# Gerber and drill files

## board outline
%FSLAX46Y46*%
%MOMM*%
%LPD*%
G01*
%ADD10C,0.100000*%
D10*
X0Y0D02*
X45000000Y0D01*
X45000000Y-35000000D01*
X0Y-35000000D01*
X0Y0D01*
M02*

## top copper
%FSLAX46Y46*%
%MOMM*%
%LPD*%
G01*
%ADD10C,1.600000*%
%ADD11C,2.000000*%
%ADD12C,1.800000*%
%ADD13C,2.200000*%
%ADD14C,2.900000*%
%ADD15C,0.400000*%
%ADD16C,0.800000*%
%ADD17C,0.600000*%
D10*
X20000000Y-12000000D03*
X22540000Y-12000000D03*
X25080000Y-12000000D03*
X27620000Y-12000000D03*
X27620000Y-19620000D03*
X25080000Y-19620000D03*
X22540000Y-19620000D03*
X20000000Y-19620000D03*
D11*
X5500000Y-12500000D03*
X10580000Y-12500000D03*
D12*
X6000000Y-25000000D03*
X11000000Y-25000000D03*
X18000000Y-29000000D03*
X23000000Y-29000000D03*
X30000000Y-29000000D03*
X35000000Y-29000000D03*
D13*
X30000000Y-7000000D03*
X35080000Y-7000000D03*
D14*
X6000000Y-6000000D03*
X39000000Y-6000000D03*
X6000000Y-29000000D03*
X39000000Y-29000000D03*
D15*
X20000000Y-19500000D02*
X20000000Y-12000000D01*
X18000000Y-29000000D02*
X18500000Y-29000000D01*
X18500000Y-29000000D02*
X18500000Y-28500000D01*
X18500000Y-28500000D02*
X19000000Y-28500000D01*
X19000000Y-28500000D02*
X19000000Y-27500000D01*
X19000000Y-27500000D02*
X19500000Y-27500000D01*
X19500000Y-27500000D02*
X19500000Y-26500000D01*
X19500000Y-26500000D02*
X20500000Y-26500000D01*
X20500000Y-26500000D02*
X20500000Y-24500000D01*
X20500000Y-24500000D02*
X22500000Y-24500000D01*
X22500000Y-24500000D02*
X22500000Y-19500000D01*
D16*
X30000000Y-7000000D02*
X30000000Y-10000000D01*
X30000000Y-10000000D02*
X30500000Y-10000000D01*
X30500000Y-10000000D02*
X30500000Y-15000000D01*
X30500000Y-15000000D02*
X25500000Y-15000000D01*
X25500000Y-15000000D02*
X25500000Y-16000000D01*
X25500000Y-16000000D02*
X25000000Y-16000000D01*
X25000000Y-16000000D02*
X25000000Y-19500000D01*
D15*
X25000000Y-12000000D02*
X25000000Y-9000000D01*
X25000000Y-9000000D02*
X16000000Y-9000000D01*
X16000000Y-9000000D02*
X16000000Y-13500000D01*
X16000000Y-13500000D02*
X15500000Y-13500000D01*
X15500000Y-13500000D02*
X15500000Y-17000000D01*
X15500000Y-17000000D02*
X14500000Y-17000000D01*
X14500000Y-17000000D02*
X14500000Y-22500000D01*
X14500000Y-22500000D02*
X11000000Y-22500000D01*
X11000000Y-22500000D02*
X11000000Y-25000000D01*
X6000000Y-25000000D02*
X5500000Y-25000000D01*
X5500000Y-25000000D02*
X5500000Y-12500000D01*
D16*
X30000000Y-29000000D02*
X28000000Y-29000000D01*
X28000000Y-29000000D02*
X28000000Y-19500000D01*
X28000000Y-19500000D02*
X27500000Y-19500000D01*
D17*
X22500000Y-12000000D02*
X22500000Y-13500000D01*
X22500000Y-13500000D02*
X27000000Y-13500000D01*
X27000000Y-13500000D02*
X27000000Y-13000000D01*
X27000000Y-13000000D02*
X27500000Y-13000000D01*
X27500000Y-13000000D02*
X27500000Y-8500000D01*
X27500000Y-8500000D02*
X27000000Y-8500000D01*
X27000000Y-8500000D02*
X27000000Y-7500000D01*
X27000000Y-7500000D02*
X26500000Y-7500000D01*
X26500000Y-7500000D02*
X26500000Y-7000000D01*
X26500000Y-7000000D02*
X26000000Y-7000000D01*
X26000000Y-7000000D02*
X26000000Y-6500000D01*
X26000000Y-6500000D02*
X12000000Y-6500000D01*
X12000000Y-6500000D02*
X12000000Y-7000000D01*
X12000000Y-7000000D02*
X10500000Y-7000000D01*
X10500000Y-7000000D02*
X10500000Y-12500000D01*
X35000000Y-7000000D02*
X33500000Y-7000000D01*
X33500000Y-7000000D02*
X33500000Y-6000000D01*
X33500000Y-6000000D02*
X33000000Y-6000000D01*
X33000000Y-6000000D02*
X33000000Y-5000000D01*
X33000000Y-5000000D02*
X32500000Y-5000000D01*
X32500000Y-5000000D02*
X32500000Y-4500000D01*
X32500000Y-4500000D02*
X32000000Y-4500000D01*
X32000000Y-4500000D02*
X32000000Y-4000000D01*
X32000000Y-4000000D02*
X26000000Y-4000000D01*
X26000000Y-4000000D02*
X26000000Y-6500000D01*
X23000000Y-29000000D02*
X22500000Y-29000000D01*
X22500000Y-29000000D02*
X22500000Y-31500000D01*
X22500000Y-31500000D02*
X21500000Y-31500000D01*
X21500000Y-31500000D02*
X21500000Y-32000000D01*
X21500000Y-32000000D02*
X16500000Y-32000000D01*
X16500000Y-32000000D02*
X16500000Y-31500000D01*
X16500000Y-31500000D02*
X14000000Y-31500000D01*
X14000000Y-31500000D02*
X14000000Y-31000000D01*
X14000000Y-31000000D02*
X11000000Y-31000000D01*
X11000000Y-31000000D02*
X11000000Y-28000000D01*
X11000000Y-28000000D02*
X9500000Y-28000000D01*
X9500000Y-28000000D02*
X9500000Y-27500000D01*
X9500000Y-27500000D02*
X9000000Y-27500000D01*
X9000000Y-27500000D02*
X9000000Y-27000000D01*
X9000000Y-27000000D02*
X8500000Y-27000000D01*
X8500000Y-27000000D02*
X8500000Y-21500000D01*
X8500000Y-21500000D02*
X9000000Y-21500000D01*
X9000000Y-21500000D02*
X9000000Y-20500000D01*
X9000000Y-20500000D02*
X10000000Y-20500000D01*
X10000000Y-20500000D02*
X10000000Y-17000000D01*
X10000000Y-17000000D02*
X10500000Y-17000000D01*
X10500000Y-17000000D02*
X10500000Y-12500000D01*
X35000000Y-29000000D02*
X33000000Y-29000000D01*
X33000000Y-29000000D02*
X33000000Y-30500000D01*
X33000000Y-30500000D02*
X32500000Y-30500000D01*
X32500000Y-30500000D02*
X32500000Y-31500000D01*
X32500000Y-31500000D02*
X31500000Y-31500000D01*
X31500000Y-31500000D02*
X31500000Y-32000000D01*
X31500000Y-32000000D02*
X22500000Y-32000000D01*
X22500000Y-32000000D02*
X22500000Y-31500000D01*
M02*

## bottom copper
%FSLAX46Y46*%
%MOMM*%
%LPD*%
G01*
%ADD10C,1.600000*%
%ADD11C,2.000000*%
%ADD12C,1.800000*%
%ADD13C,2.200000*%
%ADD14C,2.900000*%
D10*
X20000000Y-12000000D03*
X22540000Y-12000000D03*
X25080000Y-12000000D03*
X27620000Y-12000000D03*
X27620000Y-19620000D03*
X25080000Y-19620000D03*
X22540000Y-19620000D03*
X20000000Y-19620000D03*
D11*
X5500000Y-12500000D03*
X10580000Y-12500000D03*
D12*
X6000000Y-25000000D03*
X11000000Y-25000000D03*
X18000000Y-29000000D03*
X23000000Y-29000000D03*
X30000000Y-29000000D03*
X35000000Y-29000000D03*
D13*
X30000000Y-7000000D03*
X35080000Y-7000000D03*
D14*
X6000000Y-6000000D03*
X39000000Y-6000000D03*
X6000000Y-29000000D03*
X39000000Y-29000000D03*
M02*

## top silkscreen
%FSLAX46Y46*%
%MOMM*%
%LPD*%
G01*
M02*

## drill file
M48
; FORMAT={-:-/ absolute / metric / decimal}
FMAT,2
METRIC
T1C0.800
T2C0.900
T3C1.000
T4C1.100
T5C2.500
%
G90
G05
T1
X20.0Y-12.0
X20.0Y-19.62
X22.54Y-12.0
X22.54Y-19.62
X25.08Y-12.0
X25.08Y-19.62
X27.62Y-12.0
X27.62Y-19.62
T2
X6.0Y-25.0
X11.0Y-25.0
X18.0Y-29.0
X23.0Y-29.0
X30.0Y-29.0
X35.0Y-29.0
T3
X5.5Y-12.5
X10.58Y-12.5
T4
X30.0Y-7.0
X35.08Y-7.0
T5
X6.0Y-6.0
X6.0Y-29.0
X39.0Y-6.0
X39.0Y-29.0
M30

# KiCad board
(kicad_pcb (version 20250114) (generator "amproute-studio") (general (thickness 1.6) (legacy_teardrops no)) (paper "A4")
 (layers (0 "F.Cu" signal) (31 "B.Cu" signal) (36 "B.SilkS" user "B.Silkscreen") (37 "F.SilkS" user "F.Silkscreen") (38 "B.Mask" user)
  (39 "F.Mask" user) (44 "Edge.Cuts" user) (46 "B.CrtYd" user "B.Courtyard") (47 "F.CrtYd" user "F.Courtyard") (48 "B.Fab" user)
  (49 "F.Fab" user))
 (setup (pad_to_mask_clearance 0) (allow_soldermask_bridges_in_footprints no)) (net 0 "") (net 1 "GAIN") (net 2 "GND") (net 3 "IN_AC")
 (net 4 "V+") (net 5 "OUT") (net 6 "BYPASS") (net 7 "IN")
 (gr_rect (start 0 0) (end 45.0000 35.0000) (stroke (width 0.1) (type default)) (fill none) (layer "Edge.Cuts"))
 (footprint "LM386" (layer "F.Cu") (at 18.0000 10.0000)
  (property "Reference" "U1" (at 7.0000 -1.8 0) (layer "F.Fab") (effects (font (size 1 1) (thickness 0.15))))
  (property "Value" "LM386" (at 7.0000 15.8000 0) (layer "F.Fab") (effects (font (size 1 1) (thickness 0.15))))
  (pad "1" thru_hole circle (at 2.0000 2.0000) (size 1.6000 1.6000) (drill 0.8000) (layers "*.Cu" "*.Mask") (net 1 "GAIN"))
  (pad "2" thru_hole circle (at 4.5400 2.0000) (size 1.6000 1.6000) (drill 0.8000) (layers "*.Cu" "*.Mask") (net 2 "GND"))
  (pad "3" thru_hole circle (at 7.0800 2.0000) (size 1.6000 1.6000) (drill 0.8000) (layers "*.Cu" "*.Mask") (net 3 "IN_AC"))
  (pad "4" thru_hole circle (at 9.6200 2.0000) (size 1.6000 1.6000) (drill 0.8000) (layers "*.Cu" "*.Mask") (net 2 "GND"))
  (pad "5" thru_hole circle (at 9.6200 9.6200) (size 1.6000 1.6000) (drill 0.8000) (layers "*.Cu" "*.Mask") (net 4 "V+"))
  (pad "6" thru_hole circle (at 7.0800 9.6200) (size 1.6000 1.6000) (drill 0.8000) (layers "*.Cu" "*.Mask") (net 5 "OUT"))
  (pad "7" thru_hole circle (at 4.5400 9.6200) (size 1.6000 1.6000) (drill 0.8000) (layers "*.Cu" "*.Mask") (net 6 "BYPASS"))
  (pad "8" thru_hole circle (at 2.0000 9.6200) (size 1.6000 1.6000) (drill 0.8000) (layers "*.Cu" "*.Mask") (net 1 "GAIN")))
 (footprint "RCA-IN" (layer "F.Cu") (at 3.0000 8.0000)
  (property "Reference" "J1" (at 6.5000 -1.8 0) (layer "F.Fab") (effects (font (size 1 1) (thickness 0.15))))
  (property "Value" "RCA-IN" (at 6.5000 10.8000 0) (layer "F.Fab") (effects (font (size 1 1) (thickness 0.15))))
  (pad "1" thru_hole circle (at 2.5000 4.5000) (size 2.0000 2.0000) (drill 1.0000) (layers "*.Cu" "*.Mask") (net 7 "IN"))
  (pad "2" thru_hole circle (at 7.5800 4.5000) (size 2.0000 2.0000) (drill 1.0000) (layers "*.Cu" "*.Mask") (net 2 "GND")))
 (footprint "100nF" (layer "F.Cu") (at 4.0000 22.0000)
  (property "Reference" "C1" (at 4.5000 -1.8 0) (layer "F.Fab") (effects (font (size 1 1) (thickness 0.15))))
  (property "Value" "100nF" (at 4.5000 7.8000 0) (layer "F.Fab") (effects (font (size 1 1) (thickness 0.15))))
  (pad "1" thru_hole circle (at 2.0000 3.0000) (size 1.8000 1.8000) (drill 0.9000) (layers "*.Cu" "*.Mask") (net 7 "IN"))
  (pad "2" thru_hole circle (at 7.0000 3.0000) (size 1.8000 1.8000) (drill 0.9000) (layers "*.Cu" "*.Mask") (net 3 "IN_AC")))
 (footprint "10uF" (layer "F.Cu") (at 16.0000 26.0000)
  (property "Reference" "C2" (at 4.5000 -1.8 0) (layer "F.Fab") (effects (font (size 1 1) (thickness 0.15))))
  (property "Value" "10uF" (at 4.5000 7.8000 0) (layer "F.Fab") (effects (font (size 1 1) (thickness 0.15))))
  (pad "1" thru_hole circle (at 2.0000 3.0000) (size 1.8000 1.8000) (drill 0.9000) (layers "*.Cu" "*.Mask") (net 6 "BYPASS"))
  (pad "2" thru_hole circle (at 7.0000 3.0000) (size 1.8000 1.8000) (drill 0.9000) (layers "*.Cu" "*.Mask") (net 2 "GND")))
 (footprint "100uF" (layer "F.Cu") (at 28.0000 26.0000)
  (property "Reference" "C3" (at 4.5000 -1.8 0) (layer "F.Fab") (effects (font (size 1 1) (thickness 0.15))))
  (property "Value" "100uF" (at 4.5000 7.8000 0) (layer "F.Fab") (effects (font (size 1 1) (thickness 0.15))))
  (pad "1" thru_hole circle (at 2.0000 3.0000) (size 1.8000 1.8000) (drill 0.9000) (layers "*.Cu" "*.Mask") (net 4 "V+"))
  (pad "2" thru_hole circle (at 7.0000 3.0000) (size 1.8000 1.8000) (drill 0.9000) (layers "*.Cu" "*.Mask") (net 2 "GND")))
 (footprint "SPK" (layer "F.Cu") (at 28.0000 3.0000)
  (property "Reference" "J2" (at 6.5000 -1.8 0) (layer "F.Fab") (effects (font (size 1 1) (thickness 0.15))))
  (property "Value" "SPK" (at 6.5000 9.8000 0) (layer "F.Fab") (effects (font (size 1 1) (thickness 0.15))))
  (pad "1" thru_hole circle (at 2.0000 4.0000) (size 2.2000 2.2000) (drill 1.1000) (layers "*.Cu" "*.Mask") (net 5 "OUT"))
  (pad "2" thru_hole circle (at 7.0800 4.0000) (size 2.2000 2.2000) (drill 1.1000) (layers "*.Cu" "*.Mask") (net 2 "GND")))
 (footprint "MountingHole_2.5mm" (layer "F.Cu") (at 6.0000 6.0000)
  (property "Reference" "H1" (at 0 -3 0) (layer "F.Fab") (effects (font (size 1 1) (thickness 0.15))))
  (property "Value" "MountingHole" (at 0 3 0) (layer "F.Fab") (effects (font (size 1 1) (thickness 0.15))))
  (pad "" np_thru_hole circle (at 0 0) (size 2.9000 2.9000) (drill 2.5000) (layers "*.Cu" "*.Mask")))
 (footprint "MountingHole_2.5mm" (layer "F.Cu") (at 39.0000 6.0000)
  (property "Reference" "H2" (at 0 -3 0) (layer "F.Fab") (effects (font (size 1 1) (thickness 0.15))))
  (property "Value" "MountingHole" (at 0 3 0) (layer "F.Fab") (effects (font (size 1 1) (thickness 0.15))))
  (pad "" np_thru_hole circle (at 0 0) (size 2.9000 2.9000) (drill 2.5000) (layers "*.Cu" "*.Mask")))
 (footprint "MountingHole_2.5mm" (layer "F.Cu") (at 6.0000 29.0000)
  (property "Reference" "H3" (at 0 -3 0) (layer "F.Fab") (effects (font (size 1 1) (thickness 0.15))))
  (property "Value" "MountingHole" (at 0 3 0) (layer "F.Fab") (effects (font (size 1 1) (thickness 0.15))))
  (pad "" np_thru_hole circle (at 0 0) (size 2.9000 2.9000) (drill 2.5000) (layers "*.Cu" "*.Mask")))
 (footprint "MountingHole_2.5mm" (layer "F.Cu") (at 39.0000 29.0000)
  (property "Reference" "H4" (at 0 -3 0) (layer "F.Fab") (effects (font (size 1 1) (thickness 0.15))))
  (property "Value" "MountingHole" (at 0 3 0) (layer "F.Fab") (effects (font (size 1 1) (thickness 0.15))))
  (pad "" np_thru_hole circle (at 0 0) (size 2.9000 2.9000) (drill 2.5000) (layers "*.Cu" "*.Mask")))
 (segment (start 20.0000 19.5000) (end 20.0000 12.0000) (width 0.4000) (layer "F.Cu") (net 1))
 (segment (start 18.0000 29.0000) (end 18.5000 29.0000) (width 0.4000) (layer "F.Cu") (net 6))
 (segment (start 18.5000 29.0000) (end 18.5000 28.5000) (width 0.4000) (layer "F.Cu") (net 6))
 (segment (start 18.5000 28.5000) (end 19.0000 28.5000) (width 0.4000) (layer "F.Cu") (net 6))
 (segment (start 19.0000 28.5000) (end 19.0000 27.5000) (width 0.4000) (layer "F.Cu") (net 6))
 (segment (start 19.0000 27.5000) (end 19.5000 27.5000) (width 0.4000) (layer "F.Cu") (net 6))
 (segment (start 19.5000 27.5000) (end 19.5000 26.5000) (width 0.4000) (layer "F.Cu") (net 6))
 (segment (start 19.5000 26.5000) (end 20.5000 26.5000) (width 0.4000) (layer "F.Cu") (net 6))
 (segment (start 20.5000 26.5000) (end 20.5000 24.5000) (width 0.4000) (layer "F.Cu") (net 6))
 (segment (start 20.5000 24.5000) (end 22.5000 24.5000) (width 0.4000) (layer "F.Cu") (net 6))
 (segment (start 22.5000 24.5000) (end 22.5000 19.5000) (width 0.4000) (layer "F.Cu") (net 6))
 (segment (start 30.0000 7.0000) (end 30.0000 10.0000) (width 0.8000) (layer "F.Cu") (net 5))
 (segment (start 30.0000 10.0000) (end 30.5000 10.0000) (width 0.8000) (layer "F.Cu") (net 5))
 (segment (start 30.5000 10.0000) (end 30.5000 15.0000) (width 0.8000) (layer "F.Cu") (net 5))
 (segment (start 30.5000 15.0000) (end 25.5000 15.0000) (width 0.8000) (layer "F.Cu") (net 5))
 (segment (start 25.5000 15.0000) (end 25.5000 16.0000) (width 0.8000) (layer "F.Cu") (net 5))
 (segment (start 25.5000 16.0000) (end 25.0000 16.0000) (width 0.8000) (layer "F.Cu") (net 5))
 (segment (start 25.0000 16.0000) (end 25.0000 19.5000) (width 0.8000) (layer "F.Cu") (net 5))
 (segment (start 25.0000 12.0000) (end 25.0000 9.0000) (width 0.4000) (layer "F.Cu") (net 3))
 (segment (start 25.0000 9.0000) (end 16.0000 9.0000) (width 0.4000) (layer "F.Cu") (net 3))
 (segment (start 16.0000 9.0000) (end 16.0000 13.5000) (width 0.4000) (layer "F.Cu") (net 3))
 (segment (start 16.0000 13.5000) (end 15.5000 13.5000) (width 0.4000) (layer "F.Cu") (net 3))
 (segment (start 15.5000 13.5000) (end 15.5000 17.0000) (width 0.4000) (layer "F.Cu") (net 3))
 (segment (start 15.5000 17.0000) (end 14.5000 17.0000) (width 0.4000) (layer "F.Cu") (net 3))
 (segment (start 14.5000 17.0000) (end 14.5000 22.5000) (width 0.4000) (layer "F.Cu") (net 3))
 (segment (start 14.5000 22.5000) (end 11.0000 22.5000) (width 0.4000) (layer "F.Cu") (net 3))
 (segment (start 11.0000 22.5000) (end 11.0000 25.0000) (width 0.4000) (layer "F.Cu") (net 3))
 (segment (start 6.0000 25.0000) (end 5.5000 25.0000) (width 0.4000) (layer "F.Cu") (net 7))
 (segment (start 5.5000 25.0000) (end 5.5000 12.5000) (width 0.4000) (layer "F.Cu") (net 7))
 (segment (start 30.0000 29.0000) (end 28.0000 29.0000) (width 0.8000) (layer "F.Cu") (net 4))
 (segment (start 28.0000 29.0000) (end 28.0000 19.5000) (width 0.8000) (layer "F.Cu") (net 4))
 (segment (start 28.0000 19.5000) (end 27.5000 19.5000) (width 0.8000) (layer "F.Cu") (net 4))
 (segment (start 22.5000 12.0000) (end 22.5000 13.5000) (width 0.6000) (layer "F.Cu") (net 2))
 (segment (start 22.5000 13.5000) (end 27.0000 13.5000) (width 0.6000) (layer "F.Cu") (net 2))
 (segment (start 27.0000 13.5000) (end 27.0000 13.0000) (width 0.6000) (layer "F.Cu") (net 2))
 (segment (start 27.0000 13.0000) (end 27.5000 13.0000) (width 0.6000) (layer "F.Cu") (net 2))
 (segment (start 27.5000 13.0000) (end 27.5000 8.5000) (width 0.6000) (layer "F.Cu") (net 2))
 (segment (start 27.5000 8.5000) (end 27.0000 8.5000) (width 0.6000) (layer "F.Cu") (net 2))
 (segment (start 27.0000 8.5000) (end 27.0000 7.5000) (width 0.6000) (layer "F.Cu") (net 2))
 (segment (start 27.0000 7.5000) (end 26.5000 7.5000) (width 0.6000) (layer "F.Cu") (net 2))
 (segment (start 26.5000 7.5000) (end 26.5000 7.0000) (width 0.6000) (layer "F.Cu") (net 2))
 (segment (start 26.5000 7.0000) (end 26.0000 7.0000) (width 0.6000) (layer "F.Cu") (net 2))
 (segment (start 26.0000 7.0000) (end 26.0000 6.5000) (width 0.6000) (layer "F.Cu") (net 2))
 (segment (start 26.0000 6.5000) (end 12.0000 6.5000) (width 0.6000) (layer "F.Cu") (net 2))
 (segment (start 12.0000 6.5000) (end 12.0000 7.0000) (width 0.6000) (layer "F.Cu") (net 2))
 (segment (start 12.0000 7.0000) (end 10.5000 7.0000) (width 0.6000) (layer "F.Cu") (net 2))
 (segment (start 10.5000 7.0000) (end 10.5000 12.5000) (width 0.6000) (layer "F.Cu") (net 2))
 (segment (start 35.0000 7.0000) (end 33.5000 7.0000) (width 0.6000) (layer "F.Cu") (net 2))
 (segment (start 33.5000 7.0000) (end 33.5000 6.0000) (width 0.6000) (layer "F.Cu") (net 2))
 (segment (start 33.5000 6.0000) (end 33.0000 6.0000) (width 0.6000) (layer "F.Cu") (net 2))
 (segment (start 33.0000 6.0000) (end 33.0000 5.0000) (width 0.6000) (layer "F.Cu") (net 2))
 (segment (start 33.0000 5.0000) (end 32.5000 5.0000) (width 0.6000) (layer "F.Cu") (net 2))
 (segment (start 32.5000 5.0000) (end 32.5000 4.5000) (width 0.6000) (layer "F.Cu") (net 2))
 (segment (start 32.5000 4.5000) (end 32.0000 4.5000) (width 0.6000) (layer "F.Cu") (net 2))
 (segment (start 32.0000 4.5000) (end 32.0000 4.0000) (width 0.6000) (layer "F.Cu") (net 2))
 (segment (start 32.0000 4.0000) (end 26.0000 4.0000) (width 0.6000) (layer "F.Cu") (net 2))
 (segment (start 26.0000 4.0000) (end 26.0000 6.5000) (width 0.6000) (layer "F.Cu") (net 2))
 (segment (start 23.0000 29.0000) (end 22.5000 29.0000) (width 0.6000) (layer "F.Cu") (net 2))
 (segment (start 22.5000 29.0000) (end 22.5000 31.5000) (width 0.6000) (layer "F.Cu") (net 2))
 (segment (start 22.5000 31.5000) (end 21.5000 31.5000) (width 0.6000) (layer "F.Cu") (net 2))
 (segment (start 21.5000 31.5000) (end 21.5000 32.0000) (width 0.6000) (layer "F.Cu") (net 2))
 (segment (start 21.5000 32.0000) (end 16.5000 32.0000) (width 0.6000) (layer "F.Cu") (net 2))
 (segment (start 16.5000 32.0000) (end 16.5000 31.5000) (width 0.6000) (layer "F.Cu") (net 2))
 (segment (start 16.5000 31.5000) (end 14.0000 31.5000) (width 0.6000) (layer "F.Cu") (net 2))
 (segment (start 14.0000 31.5000) (end 14.0000 31.0000) (width 0.6000) (layer "F.Cu") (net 2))
 (segment (start 14.0000 31.0000) (end 11.0000 31.0000) (width 0.6000) (layer "F.Cu") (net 2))
 (segment (start 11.0000 31.0000) (end 11.0000 28.0000) (width 0.6000) (layer "F.Cu") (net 2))
 (segment (start 11.0000 28.0000) (end 9.5000 28.0000) (width 0.6000) (layer "F.Cu") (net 2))
 (segment (start 9.5000 28.0000) (end 9.5000 27.5000) (width 0.6000) (layer "F.Cu") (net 2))
 (segment (start 9.5000 27.5000) (end 9.0000 27.5000) (width 0.6000) (layer "F.Cu") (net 2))
 (segment (start 9.0000 27.5000) (end 9.0000 27.0000) (width 0.6000) (layer "F.Cu") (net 2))
 (segment (start 9.0000 27.0000) (end 8.5000 27.0000) (width 0.6000) (layer "F.Cu") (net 2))
 (segment (start 8.5000 27.0000) (end 8.5000 21.5000) (width 0.6000) (layer "F.Cu") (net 2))
 (segment (start 8.5000 21.5000) (end 9.0000 21.5000) (width 0.6000) (layer "F.Cu") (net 2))
 (segment (start 9.0000 21.5000) (end 9.0000 20.5000) (width 0.6000) (layer "F.Cu") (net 2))
 (segment (start 9.0000 20.5000) (end 10.0000 20.5000) (width 0.6000) (layer "F.Cu") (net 2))
 (segment (start 10.0000 20.5000) (end 10.0000 17.0000) (width 0.6000) (layer "F.Cu") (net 2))
 (segment (start 10.0000 17.0000) (end 10.5000 17.0000) (width 0.6000) (layer "F.Cu") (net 2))
 (segment (start 10.5000 17.0000) (end 10.5000 12.5000) (width 0.6000) (layer "F.Cu") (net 2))
 (segment (start 35.0000 29.0000) (end 33.0000 29.0000) (width 0.6000) (layer "F.Cu") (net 2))
 (segment (start 33.0000 29.0000) (end 33.0000 30.5000) (width 0.6000) (layer "F.Cu") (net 2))
 (segment (start 33.0000 30.5000) (end 32.5000 30.5000) (width 0.6000) (layer "F.Cu") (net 2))
 (segment (start 32.5000 30.5000) (end 32.5000 31.5000) (width 0.6000) (layer "F.Cu") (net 2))
 (segment (start 32.5000 31.5000) (end 31.5000 31.5000) (width 0.6000) (layer "F.Cu") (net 2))
 (segment (start 31.5000 31.5000) (end 31.5000 32.0000) (width 0.6000) (layer "F.Cu") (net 2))
 (segment (start 31.5000 32.0000) (end 22.5000 32.0000) (width 0.6000) (layer "F.Cu") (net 2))
 (segment (start 22.5000 32.0000) (end 22.5000 31.5000) (width 0.6000) (layer "F.Cu") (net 2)))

